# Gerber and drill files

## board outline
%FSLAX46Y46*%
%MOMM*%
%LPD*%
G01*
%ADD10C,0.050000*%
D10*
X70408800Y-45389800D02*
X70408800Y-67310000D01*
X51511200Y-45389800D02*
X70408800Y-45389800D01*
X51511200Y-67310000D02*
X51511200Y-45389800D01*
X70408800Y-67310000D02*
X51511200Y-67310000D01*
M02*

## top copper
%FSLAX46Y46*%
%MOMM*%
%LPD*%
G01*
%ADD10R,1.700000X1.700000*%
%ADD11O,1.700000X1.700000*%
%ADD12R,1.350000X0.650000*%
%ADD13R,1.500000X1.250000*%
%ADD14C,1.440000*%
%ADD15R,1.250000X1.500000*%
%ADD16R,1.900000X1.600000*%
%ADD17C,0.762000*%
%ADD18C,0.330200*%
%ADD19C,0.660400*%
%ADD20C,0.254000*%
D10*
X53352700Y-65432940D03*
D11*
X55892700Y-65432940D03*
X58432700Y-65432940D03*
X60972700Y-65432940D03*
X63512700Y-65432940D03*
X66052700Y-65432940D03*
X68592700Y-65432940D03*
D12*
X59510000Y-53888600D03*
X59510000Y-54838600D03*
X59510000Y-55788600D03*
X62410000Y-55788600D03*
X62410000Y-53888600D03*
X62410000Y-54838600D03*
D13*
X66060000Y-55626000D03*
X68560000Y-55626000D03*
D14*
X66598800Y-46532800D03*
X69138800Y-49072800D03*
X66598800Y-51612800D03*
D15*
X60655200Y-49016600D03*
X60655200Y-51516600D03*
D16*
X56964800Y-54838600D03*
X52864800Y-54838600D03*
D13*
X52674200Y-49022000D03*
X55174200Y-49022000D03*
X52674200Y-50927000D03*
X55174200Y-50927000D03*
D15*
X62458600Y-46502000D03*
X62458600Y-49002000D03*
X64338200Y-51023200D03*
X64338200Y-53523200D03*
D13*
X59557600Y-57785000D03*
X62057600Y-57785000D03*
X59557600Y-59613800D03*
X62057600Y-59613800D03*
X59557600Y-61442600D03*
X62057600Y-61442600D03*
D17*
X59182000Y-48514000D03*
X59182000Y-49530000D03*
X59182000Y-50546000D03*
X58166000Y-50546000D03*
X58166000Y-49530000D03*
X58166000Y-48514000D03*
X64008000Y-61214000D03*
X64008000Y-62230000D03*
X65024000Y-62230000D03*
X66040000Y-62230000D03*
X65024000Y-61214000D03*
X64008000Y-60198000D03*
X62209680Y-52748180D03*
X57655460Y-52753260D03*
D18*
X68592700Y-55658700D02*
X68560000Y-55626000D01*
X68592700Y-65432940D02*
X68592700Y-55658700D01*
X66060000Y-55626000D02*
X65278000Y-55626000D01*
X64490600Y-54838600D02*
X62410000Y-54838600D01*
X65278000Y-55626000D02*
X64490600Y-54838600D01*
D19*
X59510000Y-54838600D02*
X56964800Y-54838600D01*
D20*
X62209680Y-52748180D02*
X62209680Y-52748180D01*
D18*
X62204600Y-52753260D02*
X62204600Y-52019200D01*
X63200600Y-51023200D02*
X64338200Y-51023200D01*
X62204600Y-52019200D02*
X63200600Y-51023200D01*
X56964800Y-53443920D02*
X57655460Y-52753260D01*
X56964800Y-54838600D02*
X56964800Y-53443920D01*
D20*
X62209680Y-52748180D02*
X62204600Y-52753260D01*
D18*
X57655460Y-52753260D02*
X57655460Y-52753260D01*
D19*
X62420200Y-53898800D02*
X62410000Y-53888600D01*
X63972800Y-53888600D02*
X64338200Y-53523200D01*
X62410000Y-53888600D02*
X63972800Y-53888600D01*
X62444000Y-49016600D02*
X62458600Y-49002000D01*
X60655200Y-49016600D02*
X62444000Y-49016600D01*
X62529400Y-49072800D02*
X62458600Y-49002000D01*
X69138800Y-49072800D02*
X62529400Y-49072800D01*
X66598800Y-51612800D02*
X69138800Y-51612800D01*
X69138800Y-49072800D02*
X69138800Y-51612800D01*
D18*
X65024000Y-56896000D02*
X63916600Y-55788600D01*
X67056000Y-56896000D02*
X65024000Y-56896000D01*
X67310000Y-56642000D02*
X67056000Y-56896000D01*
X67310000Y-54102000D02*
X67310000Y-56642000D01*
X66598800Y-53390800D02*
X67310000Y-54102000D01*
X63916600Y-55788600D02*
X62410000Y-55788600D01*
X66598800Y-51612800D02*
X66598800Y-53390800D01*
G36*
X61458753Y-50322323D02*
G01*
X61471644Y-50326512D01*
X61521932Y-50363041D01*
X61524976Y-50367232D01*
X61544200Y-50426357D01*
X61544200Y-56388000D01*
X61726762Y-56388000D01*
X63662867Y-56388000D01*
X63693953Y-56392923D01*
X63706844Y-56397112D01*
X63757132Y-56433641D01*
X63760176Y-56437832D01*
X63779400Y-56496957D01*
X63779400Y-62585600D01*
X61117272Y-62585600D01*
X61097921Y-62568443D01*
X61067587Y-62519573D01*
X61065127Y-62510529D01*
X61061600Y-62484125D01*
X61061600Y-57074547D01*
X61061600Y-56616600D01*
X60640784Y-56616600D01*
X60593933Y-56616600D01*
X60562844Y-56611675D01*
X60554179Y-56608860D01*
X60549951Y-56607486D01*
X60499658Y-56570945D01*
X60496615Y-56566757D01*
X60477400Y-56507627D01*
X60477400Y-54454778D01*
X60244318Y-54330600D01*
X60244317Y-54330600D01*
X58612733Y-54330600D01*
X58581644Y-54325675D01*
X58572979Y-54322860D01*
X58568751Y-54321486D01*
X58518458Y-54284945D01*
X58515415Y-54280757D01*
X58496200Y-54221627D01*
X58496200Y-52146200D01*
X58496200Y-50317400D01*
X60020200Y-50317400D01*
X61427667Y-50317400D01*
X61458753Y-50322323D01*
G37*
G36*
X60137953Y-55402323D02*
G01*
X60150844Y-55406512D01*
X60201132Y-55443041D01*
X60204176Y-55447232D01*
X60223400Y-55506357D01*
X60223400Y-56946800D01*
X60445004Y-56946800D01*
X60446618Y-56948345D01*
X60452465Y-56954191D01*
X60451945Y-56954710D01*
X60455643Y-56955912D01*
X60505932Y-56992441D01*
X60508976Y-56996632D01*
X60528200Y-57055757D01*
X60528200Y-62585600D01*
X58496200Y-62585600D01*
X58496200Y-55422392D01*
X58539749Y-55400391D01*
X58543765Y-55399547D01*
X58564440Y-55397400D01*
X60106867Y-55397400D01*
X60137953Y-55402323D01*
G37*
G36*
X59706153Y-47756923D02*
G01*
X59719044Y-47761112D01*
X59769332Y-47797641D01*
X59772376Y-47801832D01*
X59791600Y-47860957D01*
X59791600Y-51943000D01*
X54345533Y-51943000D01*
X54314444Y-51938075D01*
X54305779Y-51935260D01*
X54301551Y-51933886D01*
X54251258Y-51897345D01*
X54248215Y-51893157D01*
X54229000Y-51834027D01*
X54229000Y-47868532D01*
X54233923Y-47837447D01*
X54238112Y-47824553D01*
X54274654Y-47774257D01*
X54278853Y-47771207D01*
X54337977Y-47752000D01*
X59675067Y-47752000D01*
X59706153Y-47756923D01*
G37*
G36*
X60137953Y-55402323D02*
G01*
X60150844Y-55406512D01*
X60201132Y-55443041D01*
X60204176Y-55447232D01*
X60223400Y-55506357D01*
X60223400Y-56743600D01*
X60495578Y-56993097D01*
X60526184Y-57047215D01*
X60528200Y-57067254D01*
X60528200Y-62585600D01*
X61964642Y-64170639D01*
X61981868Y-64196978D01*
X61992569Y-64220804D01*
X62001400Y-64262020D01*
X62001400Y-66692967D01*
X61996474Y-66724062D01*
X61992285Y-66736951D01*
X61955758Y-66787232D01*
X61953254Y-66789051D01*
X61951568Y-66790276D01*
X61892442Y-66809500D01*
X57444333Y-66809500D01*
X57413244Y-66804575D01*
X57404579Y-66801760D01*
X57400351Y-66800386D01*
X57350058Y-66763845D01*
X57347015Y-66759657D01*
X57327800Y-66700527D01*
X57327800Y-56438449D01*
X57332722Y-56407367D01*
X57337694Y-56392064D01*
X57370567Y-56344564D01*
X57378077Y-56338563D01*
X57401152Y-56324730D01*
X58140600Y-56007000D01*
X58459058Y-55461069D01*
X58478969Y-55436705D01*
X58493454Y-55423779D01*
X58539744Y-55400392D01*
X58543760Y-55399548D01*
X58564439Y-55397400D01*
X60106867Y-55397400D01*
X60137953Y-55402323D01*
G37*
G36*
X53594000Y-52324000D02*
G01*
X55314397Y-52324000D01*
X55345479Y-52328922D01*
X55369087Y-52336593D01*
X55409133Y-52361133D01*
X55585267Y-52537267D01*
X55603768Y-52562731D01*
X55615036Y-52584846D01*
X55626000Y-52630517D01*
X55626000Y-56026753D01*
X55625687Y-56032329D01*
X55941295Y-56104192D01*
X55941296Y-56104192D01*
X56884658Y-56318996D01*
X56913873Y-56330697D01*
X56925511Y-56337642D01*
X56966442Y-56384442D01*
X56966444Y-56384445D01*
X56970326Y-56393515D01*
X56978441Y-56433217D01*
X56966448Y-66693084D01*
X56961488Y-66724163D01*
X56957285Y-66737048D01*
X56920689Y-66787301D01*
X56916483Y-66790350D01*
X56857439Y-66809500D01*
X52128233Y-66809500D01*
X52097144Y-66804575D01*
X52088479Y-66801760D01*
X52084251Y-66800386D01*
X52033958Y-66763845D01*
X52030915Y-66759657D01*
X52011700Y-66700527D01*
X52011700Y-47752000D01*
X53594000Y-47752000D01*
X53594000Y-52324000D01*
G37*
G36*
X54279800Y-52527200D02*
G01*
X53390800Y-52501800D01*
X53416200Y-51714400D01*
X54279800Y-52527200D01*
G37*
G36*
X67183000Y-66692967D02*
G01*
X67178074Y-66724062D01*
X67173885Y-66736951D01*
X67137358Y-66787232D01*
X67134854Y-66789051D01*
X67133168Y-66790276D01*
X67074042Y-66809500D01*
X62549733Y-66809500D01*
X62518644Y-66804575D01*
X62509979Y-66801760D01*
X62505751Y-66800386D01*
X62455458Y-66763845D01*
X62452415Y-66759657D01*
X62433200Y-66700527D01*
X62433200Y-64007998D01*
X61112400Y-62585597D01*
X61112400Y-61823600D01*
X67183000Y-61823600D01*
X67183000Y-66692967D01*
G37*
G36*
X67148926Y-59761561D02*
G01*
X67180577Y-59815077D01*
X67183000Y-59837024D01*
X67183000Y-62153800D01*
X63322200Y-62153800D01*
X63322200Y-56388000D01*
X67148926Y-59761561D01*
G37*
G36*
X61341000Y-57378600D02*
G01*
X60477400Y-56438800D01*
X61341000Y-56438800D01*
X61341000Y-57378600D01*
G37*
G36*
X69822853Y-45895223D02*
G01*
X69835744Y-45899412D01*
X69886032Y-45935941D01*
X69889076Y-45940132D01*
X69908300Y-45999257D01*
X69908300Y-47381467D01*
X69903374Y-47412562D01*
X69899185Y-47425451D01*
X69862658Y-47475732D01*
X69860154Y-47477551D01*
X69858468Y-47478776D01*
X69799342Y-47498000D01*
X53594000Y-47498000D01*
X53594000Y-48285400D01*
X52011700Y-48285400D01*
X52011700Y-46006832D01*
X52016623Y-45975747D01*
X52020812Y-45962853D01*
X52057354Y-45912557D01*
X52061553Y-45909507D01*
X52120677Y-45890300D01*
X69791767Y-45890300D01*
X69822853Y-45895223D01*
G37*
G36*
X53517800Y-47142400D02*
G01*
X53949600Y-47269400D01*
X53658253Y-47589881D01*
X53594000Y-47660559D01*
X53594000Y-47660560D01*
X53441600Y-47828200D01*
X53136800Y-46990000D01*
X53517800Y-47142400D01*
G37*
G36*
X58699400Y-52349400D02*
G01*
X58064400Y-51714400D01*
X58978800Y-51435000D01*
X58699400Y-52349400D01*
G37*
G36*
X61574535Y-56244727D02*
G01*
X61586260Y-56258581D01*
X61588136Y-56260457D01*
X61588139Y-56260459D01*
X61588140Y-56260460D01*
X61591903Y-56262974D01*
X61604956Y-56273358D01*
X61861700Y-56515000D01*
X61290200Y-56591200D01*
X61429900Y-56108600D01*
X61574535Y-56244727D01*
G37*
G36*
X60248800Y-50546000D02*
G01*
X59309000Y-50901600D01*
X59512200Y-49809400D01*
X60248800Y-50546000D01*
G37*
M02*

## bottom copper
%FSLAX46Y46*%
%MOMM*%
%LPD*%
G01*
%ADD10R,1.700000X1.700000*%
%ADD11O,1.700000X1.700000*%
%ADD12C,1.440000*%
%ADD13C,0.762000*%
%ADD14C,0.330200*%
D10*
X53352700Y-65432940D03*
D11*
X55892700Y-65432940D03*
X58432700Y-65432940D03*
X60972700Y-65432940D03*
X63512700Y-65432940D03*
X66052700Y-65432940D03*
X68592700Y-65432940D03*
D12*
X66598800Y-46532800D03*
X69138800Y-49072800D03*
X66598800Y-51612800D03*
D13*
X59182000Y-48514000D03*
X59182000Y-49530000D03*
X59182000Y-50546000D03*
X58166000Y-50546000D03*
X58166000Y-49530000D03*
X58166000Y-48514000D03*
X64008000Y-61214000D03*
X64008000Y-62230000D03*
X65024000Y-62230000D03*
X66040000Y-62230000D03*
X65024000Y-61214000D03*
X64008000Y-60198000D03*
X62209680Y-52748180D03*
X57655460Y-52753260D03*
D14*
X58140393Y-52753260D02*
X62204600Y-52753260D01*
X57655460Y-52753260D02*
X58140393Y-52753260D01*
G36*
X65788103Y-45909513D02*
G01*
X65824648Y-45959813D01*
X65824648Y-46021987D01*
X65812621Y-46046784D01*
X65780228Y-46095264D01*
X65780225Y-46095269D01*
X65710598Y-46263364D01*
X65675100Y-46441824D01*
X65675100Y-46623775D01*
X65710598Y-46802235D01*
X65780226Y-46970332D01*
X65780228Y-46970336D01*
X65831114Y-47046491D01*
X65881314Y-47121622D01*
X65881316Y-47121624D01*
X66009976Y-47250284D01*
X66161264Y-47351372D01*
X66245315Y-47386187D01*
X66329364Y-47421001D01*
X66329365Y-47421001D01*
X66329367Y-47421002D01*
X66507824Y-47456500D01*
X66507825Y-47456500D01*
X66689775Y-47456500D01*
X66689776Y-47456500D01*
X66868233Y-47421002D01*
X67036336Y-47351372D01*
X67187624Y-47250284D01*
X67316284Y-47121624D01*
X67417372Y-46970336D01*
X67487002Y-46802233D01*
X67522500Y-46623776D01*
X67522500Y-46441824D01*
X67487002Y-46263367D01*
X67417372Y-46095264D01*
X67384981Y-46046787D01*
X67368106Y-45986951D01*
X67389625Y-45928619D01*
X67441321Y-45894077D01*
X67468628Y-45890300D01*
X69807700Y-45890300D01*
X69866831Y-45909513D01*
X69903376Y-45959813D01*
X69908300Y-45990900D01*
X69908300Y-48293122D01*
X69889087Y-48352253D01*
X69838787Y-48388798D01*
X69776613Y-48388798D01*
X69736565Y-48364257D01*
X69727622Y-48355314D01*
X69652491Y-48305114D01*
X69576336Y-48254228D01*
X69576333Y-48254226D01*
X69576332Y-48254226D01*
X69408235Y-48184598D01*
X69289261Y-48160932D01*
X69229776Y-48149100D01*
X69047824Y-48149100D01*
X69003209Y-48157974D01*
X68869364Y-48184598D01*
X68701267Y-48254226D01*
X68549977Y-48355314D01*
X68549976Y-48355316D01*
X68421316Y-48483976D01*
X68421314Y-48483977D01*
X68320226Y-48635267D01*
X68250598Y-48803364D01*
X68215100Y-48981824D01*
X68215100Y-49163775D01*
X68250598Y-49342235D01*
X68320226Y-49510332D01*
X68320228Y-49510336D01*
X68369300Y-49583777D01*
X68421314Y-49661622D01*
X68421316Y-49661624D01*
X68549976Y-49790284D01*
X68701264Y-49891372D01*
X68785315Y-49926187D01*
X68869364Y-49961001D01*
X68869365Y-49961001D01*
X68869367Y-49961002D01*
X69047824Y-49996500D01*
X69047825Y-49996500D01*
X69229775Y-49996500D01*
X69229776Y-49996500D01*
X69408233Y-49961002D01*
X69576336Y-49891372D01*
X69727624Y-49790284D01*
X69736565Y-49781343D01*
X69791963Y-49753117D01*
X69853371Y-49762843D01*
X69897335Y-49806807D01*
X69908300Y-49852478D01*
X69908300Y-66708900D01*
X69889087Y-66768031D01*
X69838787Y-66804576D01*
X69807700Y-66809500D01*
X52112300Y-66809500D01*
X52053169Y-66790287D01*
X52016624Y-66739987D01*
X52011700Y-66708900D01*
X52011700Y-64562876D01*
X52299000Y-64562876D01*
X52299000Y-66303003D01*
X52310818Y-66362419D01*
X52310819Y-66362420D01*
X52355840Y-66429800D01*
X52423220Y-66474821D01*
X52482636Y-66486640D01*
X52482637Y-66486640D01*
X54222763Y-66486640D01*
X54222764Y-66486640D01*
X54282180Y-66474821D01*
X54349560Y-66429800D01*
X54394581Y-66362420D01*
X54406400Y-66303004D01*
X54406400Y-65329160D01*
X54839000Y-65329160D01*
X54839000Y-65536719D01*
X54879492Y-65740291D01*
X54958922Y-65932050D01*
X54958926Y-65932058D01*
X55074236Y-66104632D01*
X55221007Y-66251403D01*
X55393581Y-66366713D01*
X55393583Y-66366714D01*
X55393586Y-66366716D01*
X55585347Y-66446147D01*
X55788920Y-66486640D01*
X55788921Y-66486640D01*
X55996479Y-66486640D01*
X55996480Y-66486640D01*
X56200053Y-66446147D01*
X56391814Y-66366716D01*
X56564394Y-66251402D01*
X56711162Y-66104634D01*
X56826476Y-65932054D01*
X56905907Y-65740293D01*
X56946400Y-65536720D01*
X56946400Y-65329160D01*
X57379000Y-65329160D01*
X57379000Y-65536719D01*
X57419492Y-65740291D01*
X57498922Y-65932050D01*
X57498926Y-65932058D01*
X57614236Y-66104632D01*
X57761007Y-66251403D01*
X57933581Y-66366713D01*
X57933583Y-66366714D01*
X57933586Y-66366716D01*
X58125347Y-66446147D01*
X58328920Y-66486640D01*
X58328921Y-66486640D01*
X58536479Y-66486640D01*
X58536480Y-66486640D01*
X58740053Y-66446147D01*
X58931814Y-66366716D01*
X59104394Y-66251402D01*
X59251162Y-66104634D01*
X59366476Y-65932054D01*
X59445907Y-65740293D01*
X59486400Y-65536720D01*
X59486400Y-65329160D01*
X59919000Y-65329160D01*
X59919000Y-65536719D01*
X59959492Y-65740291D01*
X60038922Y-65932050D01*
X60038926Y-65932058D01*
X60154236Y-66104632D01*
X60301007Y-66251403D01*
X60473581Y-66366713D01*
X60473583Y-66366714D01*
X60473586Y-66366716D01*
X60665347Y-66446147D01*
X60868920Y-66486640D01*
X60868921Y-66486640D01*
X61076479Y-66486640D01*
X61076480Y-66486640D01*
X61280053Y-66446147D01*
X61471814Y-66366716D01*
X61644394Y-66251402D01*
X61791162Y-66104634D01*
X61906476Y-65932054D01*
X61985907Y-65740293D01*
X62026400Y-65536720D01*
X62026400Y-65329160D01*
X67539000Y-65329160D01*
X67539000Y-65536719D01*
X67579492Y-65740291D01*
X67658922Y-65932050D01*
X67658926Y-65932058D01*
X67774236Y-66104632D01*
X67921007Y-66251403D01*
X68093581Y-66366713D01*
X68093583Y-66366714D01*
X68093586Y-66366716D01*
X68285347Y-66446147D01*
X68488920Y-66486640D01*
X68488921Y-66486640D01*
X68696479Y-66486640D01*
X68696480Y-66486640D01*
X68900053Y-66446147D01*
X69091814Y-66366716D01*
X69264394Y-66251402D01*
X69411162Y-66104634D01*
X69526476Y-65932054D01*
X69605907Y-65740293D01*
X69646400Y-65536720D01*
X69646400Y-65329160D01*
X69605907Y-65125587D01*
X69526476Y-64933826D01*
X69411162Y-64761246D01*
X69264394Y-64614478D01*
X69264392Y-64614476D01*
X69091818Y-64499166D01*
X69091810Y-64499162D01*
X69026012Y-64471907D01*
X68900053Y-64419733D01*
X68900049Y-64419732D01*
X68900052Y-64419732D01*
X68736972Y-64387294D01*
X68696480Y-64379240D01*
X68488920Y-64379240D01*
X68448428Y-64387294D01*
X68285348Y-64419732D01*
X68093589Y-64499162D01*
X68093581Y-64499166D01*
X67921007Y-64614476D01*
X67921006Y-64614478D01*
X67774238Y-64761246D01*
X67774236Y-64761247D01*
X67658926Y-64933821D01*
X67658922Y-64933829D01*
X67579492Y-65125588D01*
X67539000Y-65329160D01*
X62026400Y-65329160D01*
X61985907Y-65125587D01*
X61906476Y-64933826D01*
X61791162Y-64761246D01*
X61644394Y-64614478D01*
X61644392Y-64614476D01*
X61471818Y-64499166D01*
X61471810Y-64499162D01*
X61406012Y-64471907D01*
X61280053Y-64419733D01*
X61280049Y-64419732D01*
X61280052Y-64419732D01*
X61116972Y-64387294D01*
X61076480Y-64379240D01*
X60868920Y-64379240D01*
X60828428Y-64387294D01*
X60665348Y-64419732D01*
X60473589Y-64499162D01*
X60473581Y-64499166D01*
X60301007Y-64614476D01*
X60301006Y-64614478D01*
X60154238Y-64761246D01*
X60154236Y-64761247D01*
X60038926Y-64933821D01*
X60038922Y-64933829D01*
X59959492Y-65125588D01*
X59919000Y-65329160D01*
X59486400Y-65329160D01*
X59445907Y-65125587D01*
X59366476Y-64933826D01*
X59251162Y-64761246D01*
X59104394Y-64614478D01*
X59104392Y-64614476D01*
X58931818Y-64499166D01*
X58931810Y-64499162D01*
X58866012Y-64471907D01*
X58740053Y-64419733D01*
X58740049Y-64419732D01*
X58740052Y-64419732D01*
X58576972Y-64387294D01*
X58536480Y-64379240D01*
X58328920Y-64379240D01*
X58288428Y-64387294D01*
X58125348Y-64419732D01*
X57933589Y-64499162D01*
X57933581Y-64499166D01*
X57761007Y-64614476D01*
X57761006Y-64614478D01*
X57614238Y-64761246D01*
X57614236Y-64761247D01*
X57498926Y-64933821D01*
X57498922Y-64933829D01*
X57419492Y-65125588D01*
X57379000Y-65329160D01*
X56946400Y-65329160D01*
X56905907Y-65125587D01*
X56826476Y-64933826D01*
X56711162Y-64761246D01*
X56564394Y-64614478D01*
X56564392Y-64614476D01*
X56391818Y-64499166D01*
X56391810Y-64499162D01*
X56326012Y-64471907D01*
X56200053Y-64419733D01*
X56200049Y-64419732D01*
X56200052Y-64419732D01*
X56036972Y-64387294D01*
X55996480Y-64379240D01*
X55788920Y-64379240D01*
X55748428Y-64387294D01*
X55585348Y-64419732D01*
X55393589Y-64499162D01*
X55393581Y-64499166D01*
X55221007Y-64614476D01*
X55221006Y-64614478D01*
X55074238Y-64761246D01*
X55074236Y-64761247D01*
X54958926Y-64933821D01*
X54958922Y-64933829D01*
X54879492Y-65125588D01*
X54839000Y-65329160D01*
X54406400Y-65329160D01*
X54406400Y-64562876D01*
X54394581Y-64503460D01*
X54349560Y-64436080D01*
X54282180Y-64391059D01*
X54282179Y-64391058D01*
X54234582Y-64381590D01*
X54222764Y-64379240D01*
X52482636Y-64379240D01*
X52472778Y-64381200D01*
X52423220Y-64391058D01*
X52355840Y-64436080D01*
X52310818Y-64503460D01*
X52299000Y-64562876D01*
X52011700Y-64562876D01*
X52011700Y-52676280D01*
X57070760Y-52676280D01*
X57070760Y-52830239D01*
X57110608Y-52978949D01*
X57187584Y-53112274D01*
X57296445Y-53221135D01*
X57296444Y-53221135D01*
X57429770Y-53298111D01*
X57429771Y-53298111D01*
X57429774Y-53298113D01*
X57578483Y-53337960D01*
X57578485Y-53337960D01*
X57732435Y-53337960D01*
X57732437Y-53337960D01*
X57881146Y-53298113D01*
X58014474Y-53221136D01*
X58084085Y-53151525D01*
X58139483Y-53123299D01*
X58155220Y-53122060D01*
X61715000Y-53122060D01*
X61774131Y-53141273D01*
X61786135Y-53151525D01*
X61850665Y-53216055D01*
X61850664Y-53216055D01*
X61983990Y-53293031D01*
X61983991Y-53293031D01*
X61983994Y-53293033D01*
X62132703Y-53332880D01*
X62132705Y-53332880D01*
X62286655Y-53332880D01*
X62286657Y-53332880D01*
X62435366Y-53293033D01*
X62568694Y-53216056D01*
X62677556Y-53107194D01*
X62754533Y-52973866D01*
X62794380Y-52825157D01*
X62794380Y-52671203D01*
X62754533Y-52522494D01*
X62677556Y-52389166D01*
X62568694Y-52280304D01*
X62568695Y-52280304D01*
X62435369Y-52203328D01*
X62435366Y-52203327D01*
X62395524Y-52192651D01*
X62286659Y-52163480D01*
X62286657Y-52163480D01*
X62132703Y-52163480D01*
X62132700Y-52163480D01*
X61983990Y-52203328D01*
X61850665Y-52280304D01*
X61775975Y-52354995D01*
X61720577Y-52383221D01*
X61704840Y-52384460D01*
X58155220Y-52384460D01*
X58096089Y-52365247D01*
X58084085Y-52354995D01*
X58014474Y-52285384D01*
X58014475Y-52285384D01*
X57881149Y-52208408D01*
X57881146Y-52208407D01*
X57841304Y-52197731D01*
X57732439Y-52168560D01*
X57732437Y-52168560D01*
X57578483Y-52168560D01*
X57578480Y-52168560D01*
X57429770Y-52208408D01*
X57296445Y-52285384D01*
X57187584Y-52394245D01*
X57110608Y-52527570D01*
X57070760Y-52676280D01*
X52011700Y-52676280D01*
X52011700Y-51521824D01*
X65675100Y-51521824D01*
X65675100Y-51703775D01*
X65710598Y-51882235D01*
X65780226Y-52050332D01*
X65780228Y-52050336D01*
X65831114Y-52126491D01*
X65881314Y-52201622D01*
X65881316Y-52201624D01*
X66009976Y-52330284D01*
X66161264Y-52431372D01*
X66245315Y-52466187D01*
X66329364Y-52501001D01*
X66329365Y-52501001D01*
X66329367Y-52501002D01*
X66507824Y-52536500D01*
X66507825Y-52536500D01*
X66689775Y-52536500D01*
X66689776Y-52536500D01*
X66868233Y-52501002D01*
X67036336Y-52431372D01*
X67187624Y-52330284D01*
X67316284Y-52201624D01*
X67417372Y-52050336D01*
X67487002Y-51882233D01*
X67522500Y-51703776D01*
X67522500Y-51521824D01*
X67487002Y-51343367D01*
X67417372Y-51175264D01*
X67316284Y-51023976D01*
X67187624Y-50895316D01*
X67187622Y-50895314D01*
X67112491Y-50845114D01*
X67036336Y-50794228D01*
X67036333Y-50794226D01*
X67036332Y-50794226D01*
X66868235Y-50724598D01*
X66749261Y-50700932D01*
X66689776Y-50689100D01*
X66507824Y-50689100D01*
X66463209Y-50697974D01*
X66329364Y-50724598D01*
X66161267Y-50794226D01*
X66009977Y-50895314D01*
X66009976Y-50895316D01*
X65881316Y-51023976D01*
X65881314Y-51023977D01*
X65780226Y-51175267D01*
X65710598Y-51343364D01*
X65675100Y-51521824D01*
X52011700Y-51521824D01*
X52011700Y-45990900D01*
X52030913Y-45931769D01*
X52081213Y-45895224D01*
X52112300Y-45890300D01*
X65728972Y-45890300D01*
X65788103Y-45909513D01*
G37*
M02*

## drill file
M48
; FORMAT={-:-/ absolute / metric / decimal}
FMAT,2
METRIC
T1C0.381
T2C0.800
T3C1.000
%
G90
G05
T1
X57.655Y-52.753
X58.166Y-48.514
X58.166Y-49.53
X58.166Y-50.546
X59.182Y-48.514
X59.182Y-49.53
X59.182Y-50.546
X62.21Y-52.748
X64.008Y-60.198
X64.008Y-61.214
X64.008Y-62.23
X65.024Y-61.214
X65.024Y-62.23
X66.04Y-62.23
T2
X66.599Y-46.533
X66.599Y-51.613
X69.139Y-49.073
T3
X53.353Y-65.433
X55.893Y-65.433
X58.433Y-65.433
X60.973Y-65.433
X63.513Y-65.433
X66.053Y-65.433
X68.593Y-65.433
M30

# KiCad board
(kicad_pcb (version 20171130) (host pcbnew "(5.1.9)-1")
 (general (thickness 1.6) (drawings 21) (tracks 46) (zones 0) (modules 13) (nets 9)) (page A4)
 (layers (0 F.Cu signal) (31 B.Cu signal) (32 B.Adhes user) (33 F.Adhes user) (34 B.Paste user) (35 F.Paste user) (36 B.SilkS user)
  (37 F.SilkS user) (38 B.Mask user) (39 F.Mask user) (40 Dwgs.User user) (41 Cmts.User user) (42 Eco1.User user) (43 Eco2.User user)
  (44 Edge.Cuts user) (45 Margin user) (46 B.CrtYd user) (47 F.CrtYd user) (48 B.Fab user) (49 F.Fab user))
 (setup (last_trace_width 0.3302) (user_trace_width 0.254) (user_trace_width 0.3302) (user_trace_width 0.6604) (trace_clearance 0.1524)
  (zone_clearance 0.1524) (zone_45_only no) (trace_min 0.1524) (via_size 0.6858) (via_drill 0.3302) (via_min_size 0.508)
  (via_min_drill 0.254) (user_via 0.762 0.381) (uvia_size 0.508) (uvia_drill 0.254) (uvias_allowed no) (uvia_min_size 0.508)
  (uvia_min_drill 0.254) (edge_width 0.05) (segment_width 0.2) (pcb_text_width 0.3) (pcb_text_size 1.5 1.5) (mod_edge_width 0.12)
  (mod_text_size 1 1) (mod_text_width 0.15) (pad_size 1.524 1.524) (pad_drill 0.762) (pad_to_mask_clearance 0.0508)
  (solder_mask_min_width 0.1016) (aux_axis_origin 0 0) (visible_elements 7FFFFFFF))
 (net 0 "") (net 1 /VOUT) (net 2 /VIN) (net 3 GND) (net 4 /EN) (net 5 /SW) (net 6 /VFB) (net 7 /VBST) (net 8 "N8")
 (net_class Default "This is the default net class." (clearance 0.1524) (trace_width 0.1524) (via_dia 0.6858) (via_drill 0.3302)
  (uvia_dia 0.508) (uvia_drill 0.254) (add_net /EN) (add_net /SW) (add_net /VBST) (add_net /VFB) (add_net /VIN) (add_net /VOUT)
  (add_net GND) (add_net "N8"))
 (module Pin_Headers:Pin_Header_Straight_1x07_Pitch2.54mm (layer F.Cu) (at 53.3527 65.43294 90)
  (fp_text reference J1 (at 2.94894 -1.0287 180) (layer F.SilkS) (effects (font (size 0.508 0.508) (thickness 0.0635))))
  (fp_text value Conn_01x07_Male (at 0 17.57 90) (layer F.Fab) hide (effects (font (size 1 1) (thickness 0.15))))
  (pad 1 thru_hole rect (at 0 0 90) (size 1.7 1.7) (drill 1) (layers *.Cu *.Mask) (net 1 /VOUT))
  (pad 2 thru_hole oval (at 0 2.54 90) (size 1.7 1.7) (drill 1) (layers *.Cu *.Mask) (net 1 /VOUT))
  (pad 3 thru_hole oval (at 0 5.08 90) (size 1.7 1.7) (drill 1) (layers *.Cu *.Mask) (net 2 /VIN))
  (pad 4 thru_hole oval (at 0 7.62 90) (size 1.7 1.7) (drill 1) (layers *.Cu *.Mask) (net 2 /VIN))
  (pad 5 thru_hole oval (at 0 10.16 90) (size 1.7 1.7) (drill 1) (layers *.Cu *.Mask) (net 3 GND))
  (pad 6 thru_hole oval (at 0 12.7 90) (size 1.7 1.7) (drill 1) (layers *.Cu *.Mask) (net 3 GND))
  (pad 7 thru_hole oval (at 0 15.24 90) (size 1.7 1.7) (drill 1) (layers *.Cu *.Mask) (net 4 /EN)))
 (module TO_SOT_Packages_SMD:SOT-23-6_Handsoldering (layer F.Cu) (at 60.96 54.8386)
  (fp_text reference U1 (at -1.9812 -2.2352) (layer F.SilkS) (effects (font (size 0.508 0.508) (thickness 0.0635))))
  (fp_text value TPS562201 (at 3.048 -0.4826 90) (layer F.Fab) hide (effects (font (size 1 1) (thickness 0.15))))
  (pad 1 smd rect (at -1.45 -0.95) (size 1.35 0.65) (layers F.Cu F.Paste F.Mask) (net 3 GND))
  (pad 2 smd rect (at -1.45 0) (size 1.35 0.65) (layers F.Cu F.Paste F.Mask) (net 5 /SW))
  (pad 3 smd rect (at -1.45 0.95) (size 1.35 0.65) (layers F.Cu F.Paste F.Mask) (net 2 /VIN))
  (pad 4 smd rect (at 1.45 0.95) (size 1.35 0.65) (layers F.Cu F.Paste F.Mask) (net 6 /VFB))
  (pad 6 smd rect (at 1.45 -0.95) (size 1.35 0.65) (layers F.Cu F.Paste F.Mask) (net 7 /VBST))
  (pad 5 smd rect (at 1.45 0) (size 1.35 0.65) (layers F.Cu F.Paste F.Mask) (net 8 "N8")))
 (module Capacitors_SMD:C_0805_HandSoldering (layer F.Cu) (at 67.31 55.626)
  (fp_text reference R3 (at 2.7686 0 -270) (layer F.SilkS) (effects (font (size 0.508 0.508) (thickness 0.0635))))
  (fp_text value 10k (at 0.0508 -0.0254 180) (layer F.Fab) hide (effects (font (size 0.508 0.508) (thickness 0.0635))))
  (pad 1 smd rect (at -1.25 0) (size 1.5 1.25) (layers F.Cu F.Paste F.Mask) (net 8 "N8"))
  (pad 2 smd rect (at 1.25 0) (size 1.5 1.25) (layers F.Cu F.Paste F.Mask) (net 4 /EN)))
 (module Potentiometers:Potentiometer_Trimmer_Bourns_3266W (layer F.Cu) (at 66.5988 46.5328 90)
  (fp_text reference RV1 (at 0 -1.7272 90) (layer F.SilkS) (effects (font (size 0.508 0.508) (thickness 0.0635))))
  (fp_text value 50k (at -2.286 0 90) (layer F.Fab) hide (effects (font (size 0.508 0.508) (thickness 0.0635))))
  (pad 1 thru_hole circle (at 0 0 90) (size 1.44 1.44) (drill 0.8) (layers *.Cu *.Mask) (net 1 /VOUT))
  (pad 2 thru_hole circle (at -2.54 2.54 90) (size 1.44 1.44) (drill 0.8) (layers *.Cu *.Mask) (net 6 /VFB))
  (pad 3 thru_hole circle (at -5.08 0 90) (size 1.44 1.44) (drill 0.8) (layers *.Cu *.Mask) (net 6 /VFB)))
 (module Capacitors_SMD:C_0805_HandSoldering (layer F.Cu) (at 60.6552 50.2666 270)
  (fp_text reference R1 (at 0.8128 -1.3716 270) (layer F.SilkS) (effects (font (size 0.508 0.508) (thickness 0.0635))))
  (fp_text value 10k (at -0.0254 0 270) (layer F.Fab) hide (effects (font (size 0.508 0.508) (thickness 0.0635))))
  (pad 1 smd rect (at -1.25 0 270) (size 1.5 1.25) (layers F.Cu F.Paste F.Mask) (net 6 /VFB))
  (pad 2 smd rect (at 1.25 0 270) (size 1.5 1.25) (layers F.Cu F.Paste F.Mask) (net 3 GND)))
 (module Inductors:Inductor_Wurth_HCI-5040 (layer F.Cu) (at 54.9148 54.8386 180)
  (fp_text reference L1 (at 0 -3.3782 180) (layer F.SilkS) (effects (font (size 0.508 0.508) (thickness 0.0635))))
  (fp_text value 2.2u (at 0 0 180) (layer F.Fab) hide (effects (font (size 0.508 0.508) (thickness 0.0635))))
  (pad 1 smd rect (at -2.05 0 180) (size 1.9 1.6) (layers F.Cu F.Paste F.Mask) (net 5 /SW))
  (pad 2 smd rect (at 2.05 0 180) (size 1.9 1.6) (layers F.Cu F.Paste F.Mask) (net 1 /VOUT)))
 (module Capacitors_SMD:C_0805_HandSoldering (layer F.Cu) (at 53.9242 49.022)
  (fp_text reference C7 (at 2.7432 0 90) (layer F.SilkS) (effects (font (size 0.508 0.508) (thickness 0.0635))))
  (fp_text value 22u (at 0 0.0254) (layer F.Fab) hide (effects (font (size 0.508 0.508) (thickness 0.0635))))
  (pad 1 smd rect (at -1.25 0) (size 1.5 1.25) (layers F.Cu F.Paste F.Mask) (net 1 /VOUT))
  (pad 2 smd rect (at 1.25 0) (size 1.5 1.25) (layers F.Cu F.Paste F.Mask) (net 3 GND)))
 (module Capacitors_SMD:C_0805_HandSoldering (layer F.Cu) (at 53.9242 50.927)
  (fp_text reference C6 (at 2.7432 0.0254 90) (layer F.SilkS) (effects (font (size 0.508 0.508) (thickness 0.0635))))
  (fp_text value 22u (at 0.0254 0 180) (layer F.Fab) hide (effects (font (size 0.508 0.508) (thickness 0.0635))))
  (pad 1 smd rect (at -1.25 0) (size 1.5 1.25) (layers F.Cu F.Paste F.Mask) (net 1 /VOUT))
  (pad 2 smd rect (at 1.25 0) (size 1.5 1.25) (layers F.Cu F.Paste F.Mask) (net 3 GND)))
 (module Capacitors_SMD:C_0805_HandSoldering (layer F.Cu) (at 62.4586 47.752 270)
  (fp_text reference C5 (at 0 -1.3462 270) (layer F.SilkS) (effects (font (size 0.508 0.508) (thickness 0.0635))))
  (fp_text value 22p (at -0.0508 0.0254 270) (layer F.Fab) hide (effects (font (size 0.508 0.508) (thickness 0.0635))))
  (pad 1 smd rect (at -1.25 0 270) (size 1.5 1.25) (layers F.Cu F.Paste F.Mask) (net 1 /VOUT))
  (pad 2 smd rect (at 1.25 0 270) (size 1.5 1.25) (layers F.Cu F.Paste F.Mask) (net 6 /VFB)))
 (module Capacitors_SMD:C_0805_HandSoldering (layer F.Cu) (at 64.3382 52.2732 270)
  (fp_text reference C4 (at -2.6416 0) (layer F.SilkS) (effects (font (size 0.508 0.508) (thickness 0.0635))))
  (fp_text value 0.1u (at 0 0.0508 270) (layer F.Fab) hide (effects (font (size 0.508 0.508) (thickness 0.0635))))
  (pad 1 smd rect (at -1.25 0 270) (size 1.5 1.25) (layers F.Cu F.Paste F.Mask) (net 5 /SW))
  (pad 2 smd rect (at 1.25 0 270) (size 1.5 1.25) (layers F.Cu F.Paste F.Mask) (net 7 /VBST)))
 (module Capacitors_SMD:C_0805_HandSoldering (layer F.Cu) (at 60.8076 57.785)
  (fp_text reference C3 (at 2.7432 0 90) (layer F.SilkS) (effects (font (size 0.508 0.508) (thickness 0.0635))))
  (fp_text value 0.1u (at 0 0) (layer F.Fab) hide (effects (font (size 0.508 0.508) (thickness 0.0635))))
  (pad 1 smd rect (at -1.25 0) (size 1.5 1.25) (layers F.Cu F.Paste F.Mask) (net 2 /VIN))
  (pad 2 smd rect (at 1.25 0) (size 1.5 1.25) (layers F.Cu F.Paste F.Mask) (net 3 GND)))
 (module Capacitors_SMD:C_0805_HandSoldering (layer F.Cu) (at 60.8076 59.6138)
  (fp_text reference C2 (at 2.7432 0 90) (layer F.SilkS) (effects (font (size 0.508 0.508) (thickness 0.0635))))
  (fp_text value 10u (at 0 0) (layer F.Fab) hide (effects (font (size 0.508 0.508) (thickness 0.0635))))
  (pad 1 smd rect (at -1.25 0) (size 1.5 1.25) (layers F.Cu F.Paste F.Mask) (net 2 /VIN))
  (pad 2 smd rect (at 1.25 0) (size 1.5 1.25) (layers F.Cu F.Paste F.Mask) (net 3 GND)))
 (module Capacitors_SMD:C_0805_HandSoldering (layer F.Cu) (at 60.8076 61.4426)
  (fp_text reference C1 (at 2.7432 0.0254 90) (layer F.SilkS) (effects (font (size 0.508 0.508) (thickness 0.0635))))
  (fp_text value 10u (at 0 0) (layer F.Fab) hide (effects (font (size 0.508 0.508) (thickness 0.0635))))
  (pad 1 smd rect (at -1.25 0) (size 1.5 1.25) (layers F.Cu F.Paste F.Mask) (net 2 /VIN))
  (pad 2 smd rect (at 1.25 0) (size 1.5 1.25) (layers F.Cu F.Paste F.Mask) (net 3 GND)))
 (gr_line (start 70.4088 45.3898) (end 70.4088 67.31) (layer Edge.Cuts) (width 0.05))
 (gr_line (start 51.5112 45.3898) (end 70.4088 45.3898) (layer Edge.Cuts) (width 0.05))
 (gr_line (start 51.5112 67.31) (end 51.5112 45.3898) (layer Edge.Cuts) (width 0.05))
 (gr_line (start 70.4088 67.31) (end 51.5112 67.31) (layer Edge.Cuts) (width 0.05))
 (via (at 59.182 48.514) (size 0.762) (drill 0.381) (layers F.Cu B.Cu) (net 3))
 (via (at 59.182 49.53) (size 0.762) (drill 0.381) (layers F.Cu B.Cu) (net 3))
 (via (at 59.182 50.546) (size 0.762) (drill 0.381) (layers F.Cu B.Cu) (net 3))
 (via (at 58.166 50.546) (size 0.762) (drill 0.381) (layers F.Cu B.Cu) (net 3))
 (via (at 58.166 49.53) (size 0.762) (drill 0.381) (layers F.Cu B.Cu) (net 3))
 (via (at 58.166 48.514) (size 0.762) (drill 0.381) (layers F.Cu B.Cu) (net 3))
 (via (at 64.008 61.214) (size 0.762) (drill 0.381) (layers F.Cu B.Cu) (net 3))
 (via (at 64.008 62.23) (size 0.762) (drill 0.381) (layers F.Cu B.Cu) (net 3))
 (via (at 65.024 62.23) (size 0.762) (drill 0.381) (layers F.Cu B.Cu) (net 3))
 (via (at 66.04 62.23) (size 0.762) (drill 0.381) (layers F.Cu B.Cu) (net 3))
 (via (at 65.024 61.214) (size 0.762) (drill 0.381) (layers F.Cu B.Cu) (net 3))
 (via (at 64.008 60.198) (size 0.762) (drill 0.381) (layers F.Cu B.Cu) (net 3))
 (segment (start 68.5927 55.6587) (end 68.56 55.626) (width 0.3302) (layer F.Cu) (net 4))
 (segment (start 68.5927 65.43294) (end 68.5927 55.6587) (width 0.3302) (layer F.Cu) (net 4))
 (segment (start 66.06 55.626) (end 65.278 55.626) (width 0.3302) (layer F.Cu) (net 8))
 (segment (start 64.4906 54.8386) (end 62.41 54.8386) (width 0.3302) (layer F.Cu) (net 8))
 (segment (start 65.278 55.626) (end 64.4906 54.8386) (width 0.3302) (layer F.Cu) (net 8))
 (segment (start 59.51 54.8386) (end 56.9648 54.8386) (width 0.6604) (layer F.Cu) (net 5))
 (segment (start 62.20968 52.74818) (end 62.20968 52.74818) (width 0.254) (layer F.Cu) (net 5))
 (segment (start 62.2046 52.75326) (end 62.2046 52.0192) (width 0.3302) (layer F.Cu) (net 5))
 (segment (start 63.2006 51.0232) (end 64.3382 51.0232) (width 0.3302) (layer F.Cu) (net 5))
 (segment (start 62.2046 52.0192) (end 63.2006 51.0232) (width 0.3302) (layer F.Cu) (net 5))
 (segment (start 56.9648 53.44392) (end 57.65546 52.75326) (width 0.3302) (layer F.Cu) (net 5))
 (segment (start 56.9648 54.8386) (end 56.9648 53.44392) (width 0.3302) (layer F.Cu) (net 5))
 (segment (start 58.140393 52.75326) (end 62.2046 52.75326) (width 0.3302) (layer B.Cu) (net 5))
 (segment (start 57.65546 52.75326) (end 58.140393 52.75326) (width 0.3302) (layer B.Cu) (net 5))
 (segment (start 62.20968 52.74818) (end 62.2046 52.75326) (width 0.254) (layer F.Cu) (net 5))
 (via (at 62.20968 52.74818) (size 0.762) (drill 0.381) (layers F.Cu B.Cu) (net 5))
 (segment (start 57.65546 52.75326) (end 57.65546 52.75326) (width 0.3302) (layer F.Cu) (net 5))
 (via (at 57.65546 52.75326) (size 0.762) (drill 0.381) (layers F.Cu B.Cu) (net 5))
 (segment (start 62.4202 53.8988) (end 62.41 53.8886) (width 0.6604) (layer F.Cu) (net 7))
 (segment (start 63.9728 53.8886) (end 64.3382 53.5232) (width 0.6604) (layer F.Cu) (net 7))
 (segment (start 62.41 53.8886) (end 63.9728 53.8886) (width 0.6604) (layer F.Cu) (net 7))
 (segment (start 62.444 49.0166) (end 62.4586 49.002) (width 0.6604) (layer F.Cu) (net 6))
 (segment (start 60.6552 49.0166) (end 62.444 49.0166) (width 0.6604) (layer F.Cu) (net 6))
 (segment (start 62.5294 49.0728) (end 62.4586 49.002) (width 0.6604) (layer F.Cu) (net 6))
 (segment (start 69.1388 49.0728) (end 62.5294 49.0728) (width 0.6604) (layer F.Cu) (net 6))
 (segment (start 66.5988 51.6128) (end 69.1388 51.6128) (width 0.6604) (layer F.Cu) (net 6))
 (segment (start 69.1388 49.0728) (end 69.1388 51.6128) (width 0.6604) (layer F.Cu) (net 6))
 (segment (start 65.024 56.896) (end 63.9166 55.7886) (width 0.3302) (layer F.Cu) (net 6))
 (segment (start 67.056 56.896) (end 65.024 56.896) (width 0.3302) (layer F.Cu) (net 6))
 (segment (start 67.31 56.642) (end 67.056 56.896) (width 0.3302) (layer F.Cu) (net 6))
 (segment (start 67.31 54.102) (end 67.31 56.642) (width 0.3302) (layer F.Cu) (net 6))
 (segment (start 66.5988 53.3908) (end 67.31 54.102) (width 0.3302) (layer F.Cu) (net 6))
 (segment (start 63.9166 55.7886) (end 62.41 55.7886) (width 0.3302) (layer F.Cu) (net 6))
 (segment (start 66.5988 51.6128) (end 66.5988 53.3908) (width 0.3302) (layer F.Cu) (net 6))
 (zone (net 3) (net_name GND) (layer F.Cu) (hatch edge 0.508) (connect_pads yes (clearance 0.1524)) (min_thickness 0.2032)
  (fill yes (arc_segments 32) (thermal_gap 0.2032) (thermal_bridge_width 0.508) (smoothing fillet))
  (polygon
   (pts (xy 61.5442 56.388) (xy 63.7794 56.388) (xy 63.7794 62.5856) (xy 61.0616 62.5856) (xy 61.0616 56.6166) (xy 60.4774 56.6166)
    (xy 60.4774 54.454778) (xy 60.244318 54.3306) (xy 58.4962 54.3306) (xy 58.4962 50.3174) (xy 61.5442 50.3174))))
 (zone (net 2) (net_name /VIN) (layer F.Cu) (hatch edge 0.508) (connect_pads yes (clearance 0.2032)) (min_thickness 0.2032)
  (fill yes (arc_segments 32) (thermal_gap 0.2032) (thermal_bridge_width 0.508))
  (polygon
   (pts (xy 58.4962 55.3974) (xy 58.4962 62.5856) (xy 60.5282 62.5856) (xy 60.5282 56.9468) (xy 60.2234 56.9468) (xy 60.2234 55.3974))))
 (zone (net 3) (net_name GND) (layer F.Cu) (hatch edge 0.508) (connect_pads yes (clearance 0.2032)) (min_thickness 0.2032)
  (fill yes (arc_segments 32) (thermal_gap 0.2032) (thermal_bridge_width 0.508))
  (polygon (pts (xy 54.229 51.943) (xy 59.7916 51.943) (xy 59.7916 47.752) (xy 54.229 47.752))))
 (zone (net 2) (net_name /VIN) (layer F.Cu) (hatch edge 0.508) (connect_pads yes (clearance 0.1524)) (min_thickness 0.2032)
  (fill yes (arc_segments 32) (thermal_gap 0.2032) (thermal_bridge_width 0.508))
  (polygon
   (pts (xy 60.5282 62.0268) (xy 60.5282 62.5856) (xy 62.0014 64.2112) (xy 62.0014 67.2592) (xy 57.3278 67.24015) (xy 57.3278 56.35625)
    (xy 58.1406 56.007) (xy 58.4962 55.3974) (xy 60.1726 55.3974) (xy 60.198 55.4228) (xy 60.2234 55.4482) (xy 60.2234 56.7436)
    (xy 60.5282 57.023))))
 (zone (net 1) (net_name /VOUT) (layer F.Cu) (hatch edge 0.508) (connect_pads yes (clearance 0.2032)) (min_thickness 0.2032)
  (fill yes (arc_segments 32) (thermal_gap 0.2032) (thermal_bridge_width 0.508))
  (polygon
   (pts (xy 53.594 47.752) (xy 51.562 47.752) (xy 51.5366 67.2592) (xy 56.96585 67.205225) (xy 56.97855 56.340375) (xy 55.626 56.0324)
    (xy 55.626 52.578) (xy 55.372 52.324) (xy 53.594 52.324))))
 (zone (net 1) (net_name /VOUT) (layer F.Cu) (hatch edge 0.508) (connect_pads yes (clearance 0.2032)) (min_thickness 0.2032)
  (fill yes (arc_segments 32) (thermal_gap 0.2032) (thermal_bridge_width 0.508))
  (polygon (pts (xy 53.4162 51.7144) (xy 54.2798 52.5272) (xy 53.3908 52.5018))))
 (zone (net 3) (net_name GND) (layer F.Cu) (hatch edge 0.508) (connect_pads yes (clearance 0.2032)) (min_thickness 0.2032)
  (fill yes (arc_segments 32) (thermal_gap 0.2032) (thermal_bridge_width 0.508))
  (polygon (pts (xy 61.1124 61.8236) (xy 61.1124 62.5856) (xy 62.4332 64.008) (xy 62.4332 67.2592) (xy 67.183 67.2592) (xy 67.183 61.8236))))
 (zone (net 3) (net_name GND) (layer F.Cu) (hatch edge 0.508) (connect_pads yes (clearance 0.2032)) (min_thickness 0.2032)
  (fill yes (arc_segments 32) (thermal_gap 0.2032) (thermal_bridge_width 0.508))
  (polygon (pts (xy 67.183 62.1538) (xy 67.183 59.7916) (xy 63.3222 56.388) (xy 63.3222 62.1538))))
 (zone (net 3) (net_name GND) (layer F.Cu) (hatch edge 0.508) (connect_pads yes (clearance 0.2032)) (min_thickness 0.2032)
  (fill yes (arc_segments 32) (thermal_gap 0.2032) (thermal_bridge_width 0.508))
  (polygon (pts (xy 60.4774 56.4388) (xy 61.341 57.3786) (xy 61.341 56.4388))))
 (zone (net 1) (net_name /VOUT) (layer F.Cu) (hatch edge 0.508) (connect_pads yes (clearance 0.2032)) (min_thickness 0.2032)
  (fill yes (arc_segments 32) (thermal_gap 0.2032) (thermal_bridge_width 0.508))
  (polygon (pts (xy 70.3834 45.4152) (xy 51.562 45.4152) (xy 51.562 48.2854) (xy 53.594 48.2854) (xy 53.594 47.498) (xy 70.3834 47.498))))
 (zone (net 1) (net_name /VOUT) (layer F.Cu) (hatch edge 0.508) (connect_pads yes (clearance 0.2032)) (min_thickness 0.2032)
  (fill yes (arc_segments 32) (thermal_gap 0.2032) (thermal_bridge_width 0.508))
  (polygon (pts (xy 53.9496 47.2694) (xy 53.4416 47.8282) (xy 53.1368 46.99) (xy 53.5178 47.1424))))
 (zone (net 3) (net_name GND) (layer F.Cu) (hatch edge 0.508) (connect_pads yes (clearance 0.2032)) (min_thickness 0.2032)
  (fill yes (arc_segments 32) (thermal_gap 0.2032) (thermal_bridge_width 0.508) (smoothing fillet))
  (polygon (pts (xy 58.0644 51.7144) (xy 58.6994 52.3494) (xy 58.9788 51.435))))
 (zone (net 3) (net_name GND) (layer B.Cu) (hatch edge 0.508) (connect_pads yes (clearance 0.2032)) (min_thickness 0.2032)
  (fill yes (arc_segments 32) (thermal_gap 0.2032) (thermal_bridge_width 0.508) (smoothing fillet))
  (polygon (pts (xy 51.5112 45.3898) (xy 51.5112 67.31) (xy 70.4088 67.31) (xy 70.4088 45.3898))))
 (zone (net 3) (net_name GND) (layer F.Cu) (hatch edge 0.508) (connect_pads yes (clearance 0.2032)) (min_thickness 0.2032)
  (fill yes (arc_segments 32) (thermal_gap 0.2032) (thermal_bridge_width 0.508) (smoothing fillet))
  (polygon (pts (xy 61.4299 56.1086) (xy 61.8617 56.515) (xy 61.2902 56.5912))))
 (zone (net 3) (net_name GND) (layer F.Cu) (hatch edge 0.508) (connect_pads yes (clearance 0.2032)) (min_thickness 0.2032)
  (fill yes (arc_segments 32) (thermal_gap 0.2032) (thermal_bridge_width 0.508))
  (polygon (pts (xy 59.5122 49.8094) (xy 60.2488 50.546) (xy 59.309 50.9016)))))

